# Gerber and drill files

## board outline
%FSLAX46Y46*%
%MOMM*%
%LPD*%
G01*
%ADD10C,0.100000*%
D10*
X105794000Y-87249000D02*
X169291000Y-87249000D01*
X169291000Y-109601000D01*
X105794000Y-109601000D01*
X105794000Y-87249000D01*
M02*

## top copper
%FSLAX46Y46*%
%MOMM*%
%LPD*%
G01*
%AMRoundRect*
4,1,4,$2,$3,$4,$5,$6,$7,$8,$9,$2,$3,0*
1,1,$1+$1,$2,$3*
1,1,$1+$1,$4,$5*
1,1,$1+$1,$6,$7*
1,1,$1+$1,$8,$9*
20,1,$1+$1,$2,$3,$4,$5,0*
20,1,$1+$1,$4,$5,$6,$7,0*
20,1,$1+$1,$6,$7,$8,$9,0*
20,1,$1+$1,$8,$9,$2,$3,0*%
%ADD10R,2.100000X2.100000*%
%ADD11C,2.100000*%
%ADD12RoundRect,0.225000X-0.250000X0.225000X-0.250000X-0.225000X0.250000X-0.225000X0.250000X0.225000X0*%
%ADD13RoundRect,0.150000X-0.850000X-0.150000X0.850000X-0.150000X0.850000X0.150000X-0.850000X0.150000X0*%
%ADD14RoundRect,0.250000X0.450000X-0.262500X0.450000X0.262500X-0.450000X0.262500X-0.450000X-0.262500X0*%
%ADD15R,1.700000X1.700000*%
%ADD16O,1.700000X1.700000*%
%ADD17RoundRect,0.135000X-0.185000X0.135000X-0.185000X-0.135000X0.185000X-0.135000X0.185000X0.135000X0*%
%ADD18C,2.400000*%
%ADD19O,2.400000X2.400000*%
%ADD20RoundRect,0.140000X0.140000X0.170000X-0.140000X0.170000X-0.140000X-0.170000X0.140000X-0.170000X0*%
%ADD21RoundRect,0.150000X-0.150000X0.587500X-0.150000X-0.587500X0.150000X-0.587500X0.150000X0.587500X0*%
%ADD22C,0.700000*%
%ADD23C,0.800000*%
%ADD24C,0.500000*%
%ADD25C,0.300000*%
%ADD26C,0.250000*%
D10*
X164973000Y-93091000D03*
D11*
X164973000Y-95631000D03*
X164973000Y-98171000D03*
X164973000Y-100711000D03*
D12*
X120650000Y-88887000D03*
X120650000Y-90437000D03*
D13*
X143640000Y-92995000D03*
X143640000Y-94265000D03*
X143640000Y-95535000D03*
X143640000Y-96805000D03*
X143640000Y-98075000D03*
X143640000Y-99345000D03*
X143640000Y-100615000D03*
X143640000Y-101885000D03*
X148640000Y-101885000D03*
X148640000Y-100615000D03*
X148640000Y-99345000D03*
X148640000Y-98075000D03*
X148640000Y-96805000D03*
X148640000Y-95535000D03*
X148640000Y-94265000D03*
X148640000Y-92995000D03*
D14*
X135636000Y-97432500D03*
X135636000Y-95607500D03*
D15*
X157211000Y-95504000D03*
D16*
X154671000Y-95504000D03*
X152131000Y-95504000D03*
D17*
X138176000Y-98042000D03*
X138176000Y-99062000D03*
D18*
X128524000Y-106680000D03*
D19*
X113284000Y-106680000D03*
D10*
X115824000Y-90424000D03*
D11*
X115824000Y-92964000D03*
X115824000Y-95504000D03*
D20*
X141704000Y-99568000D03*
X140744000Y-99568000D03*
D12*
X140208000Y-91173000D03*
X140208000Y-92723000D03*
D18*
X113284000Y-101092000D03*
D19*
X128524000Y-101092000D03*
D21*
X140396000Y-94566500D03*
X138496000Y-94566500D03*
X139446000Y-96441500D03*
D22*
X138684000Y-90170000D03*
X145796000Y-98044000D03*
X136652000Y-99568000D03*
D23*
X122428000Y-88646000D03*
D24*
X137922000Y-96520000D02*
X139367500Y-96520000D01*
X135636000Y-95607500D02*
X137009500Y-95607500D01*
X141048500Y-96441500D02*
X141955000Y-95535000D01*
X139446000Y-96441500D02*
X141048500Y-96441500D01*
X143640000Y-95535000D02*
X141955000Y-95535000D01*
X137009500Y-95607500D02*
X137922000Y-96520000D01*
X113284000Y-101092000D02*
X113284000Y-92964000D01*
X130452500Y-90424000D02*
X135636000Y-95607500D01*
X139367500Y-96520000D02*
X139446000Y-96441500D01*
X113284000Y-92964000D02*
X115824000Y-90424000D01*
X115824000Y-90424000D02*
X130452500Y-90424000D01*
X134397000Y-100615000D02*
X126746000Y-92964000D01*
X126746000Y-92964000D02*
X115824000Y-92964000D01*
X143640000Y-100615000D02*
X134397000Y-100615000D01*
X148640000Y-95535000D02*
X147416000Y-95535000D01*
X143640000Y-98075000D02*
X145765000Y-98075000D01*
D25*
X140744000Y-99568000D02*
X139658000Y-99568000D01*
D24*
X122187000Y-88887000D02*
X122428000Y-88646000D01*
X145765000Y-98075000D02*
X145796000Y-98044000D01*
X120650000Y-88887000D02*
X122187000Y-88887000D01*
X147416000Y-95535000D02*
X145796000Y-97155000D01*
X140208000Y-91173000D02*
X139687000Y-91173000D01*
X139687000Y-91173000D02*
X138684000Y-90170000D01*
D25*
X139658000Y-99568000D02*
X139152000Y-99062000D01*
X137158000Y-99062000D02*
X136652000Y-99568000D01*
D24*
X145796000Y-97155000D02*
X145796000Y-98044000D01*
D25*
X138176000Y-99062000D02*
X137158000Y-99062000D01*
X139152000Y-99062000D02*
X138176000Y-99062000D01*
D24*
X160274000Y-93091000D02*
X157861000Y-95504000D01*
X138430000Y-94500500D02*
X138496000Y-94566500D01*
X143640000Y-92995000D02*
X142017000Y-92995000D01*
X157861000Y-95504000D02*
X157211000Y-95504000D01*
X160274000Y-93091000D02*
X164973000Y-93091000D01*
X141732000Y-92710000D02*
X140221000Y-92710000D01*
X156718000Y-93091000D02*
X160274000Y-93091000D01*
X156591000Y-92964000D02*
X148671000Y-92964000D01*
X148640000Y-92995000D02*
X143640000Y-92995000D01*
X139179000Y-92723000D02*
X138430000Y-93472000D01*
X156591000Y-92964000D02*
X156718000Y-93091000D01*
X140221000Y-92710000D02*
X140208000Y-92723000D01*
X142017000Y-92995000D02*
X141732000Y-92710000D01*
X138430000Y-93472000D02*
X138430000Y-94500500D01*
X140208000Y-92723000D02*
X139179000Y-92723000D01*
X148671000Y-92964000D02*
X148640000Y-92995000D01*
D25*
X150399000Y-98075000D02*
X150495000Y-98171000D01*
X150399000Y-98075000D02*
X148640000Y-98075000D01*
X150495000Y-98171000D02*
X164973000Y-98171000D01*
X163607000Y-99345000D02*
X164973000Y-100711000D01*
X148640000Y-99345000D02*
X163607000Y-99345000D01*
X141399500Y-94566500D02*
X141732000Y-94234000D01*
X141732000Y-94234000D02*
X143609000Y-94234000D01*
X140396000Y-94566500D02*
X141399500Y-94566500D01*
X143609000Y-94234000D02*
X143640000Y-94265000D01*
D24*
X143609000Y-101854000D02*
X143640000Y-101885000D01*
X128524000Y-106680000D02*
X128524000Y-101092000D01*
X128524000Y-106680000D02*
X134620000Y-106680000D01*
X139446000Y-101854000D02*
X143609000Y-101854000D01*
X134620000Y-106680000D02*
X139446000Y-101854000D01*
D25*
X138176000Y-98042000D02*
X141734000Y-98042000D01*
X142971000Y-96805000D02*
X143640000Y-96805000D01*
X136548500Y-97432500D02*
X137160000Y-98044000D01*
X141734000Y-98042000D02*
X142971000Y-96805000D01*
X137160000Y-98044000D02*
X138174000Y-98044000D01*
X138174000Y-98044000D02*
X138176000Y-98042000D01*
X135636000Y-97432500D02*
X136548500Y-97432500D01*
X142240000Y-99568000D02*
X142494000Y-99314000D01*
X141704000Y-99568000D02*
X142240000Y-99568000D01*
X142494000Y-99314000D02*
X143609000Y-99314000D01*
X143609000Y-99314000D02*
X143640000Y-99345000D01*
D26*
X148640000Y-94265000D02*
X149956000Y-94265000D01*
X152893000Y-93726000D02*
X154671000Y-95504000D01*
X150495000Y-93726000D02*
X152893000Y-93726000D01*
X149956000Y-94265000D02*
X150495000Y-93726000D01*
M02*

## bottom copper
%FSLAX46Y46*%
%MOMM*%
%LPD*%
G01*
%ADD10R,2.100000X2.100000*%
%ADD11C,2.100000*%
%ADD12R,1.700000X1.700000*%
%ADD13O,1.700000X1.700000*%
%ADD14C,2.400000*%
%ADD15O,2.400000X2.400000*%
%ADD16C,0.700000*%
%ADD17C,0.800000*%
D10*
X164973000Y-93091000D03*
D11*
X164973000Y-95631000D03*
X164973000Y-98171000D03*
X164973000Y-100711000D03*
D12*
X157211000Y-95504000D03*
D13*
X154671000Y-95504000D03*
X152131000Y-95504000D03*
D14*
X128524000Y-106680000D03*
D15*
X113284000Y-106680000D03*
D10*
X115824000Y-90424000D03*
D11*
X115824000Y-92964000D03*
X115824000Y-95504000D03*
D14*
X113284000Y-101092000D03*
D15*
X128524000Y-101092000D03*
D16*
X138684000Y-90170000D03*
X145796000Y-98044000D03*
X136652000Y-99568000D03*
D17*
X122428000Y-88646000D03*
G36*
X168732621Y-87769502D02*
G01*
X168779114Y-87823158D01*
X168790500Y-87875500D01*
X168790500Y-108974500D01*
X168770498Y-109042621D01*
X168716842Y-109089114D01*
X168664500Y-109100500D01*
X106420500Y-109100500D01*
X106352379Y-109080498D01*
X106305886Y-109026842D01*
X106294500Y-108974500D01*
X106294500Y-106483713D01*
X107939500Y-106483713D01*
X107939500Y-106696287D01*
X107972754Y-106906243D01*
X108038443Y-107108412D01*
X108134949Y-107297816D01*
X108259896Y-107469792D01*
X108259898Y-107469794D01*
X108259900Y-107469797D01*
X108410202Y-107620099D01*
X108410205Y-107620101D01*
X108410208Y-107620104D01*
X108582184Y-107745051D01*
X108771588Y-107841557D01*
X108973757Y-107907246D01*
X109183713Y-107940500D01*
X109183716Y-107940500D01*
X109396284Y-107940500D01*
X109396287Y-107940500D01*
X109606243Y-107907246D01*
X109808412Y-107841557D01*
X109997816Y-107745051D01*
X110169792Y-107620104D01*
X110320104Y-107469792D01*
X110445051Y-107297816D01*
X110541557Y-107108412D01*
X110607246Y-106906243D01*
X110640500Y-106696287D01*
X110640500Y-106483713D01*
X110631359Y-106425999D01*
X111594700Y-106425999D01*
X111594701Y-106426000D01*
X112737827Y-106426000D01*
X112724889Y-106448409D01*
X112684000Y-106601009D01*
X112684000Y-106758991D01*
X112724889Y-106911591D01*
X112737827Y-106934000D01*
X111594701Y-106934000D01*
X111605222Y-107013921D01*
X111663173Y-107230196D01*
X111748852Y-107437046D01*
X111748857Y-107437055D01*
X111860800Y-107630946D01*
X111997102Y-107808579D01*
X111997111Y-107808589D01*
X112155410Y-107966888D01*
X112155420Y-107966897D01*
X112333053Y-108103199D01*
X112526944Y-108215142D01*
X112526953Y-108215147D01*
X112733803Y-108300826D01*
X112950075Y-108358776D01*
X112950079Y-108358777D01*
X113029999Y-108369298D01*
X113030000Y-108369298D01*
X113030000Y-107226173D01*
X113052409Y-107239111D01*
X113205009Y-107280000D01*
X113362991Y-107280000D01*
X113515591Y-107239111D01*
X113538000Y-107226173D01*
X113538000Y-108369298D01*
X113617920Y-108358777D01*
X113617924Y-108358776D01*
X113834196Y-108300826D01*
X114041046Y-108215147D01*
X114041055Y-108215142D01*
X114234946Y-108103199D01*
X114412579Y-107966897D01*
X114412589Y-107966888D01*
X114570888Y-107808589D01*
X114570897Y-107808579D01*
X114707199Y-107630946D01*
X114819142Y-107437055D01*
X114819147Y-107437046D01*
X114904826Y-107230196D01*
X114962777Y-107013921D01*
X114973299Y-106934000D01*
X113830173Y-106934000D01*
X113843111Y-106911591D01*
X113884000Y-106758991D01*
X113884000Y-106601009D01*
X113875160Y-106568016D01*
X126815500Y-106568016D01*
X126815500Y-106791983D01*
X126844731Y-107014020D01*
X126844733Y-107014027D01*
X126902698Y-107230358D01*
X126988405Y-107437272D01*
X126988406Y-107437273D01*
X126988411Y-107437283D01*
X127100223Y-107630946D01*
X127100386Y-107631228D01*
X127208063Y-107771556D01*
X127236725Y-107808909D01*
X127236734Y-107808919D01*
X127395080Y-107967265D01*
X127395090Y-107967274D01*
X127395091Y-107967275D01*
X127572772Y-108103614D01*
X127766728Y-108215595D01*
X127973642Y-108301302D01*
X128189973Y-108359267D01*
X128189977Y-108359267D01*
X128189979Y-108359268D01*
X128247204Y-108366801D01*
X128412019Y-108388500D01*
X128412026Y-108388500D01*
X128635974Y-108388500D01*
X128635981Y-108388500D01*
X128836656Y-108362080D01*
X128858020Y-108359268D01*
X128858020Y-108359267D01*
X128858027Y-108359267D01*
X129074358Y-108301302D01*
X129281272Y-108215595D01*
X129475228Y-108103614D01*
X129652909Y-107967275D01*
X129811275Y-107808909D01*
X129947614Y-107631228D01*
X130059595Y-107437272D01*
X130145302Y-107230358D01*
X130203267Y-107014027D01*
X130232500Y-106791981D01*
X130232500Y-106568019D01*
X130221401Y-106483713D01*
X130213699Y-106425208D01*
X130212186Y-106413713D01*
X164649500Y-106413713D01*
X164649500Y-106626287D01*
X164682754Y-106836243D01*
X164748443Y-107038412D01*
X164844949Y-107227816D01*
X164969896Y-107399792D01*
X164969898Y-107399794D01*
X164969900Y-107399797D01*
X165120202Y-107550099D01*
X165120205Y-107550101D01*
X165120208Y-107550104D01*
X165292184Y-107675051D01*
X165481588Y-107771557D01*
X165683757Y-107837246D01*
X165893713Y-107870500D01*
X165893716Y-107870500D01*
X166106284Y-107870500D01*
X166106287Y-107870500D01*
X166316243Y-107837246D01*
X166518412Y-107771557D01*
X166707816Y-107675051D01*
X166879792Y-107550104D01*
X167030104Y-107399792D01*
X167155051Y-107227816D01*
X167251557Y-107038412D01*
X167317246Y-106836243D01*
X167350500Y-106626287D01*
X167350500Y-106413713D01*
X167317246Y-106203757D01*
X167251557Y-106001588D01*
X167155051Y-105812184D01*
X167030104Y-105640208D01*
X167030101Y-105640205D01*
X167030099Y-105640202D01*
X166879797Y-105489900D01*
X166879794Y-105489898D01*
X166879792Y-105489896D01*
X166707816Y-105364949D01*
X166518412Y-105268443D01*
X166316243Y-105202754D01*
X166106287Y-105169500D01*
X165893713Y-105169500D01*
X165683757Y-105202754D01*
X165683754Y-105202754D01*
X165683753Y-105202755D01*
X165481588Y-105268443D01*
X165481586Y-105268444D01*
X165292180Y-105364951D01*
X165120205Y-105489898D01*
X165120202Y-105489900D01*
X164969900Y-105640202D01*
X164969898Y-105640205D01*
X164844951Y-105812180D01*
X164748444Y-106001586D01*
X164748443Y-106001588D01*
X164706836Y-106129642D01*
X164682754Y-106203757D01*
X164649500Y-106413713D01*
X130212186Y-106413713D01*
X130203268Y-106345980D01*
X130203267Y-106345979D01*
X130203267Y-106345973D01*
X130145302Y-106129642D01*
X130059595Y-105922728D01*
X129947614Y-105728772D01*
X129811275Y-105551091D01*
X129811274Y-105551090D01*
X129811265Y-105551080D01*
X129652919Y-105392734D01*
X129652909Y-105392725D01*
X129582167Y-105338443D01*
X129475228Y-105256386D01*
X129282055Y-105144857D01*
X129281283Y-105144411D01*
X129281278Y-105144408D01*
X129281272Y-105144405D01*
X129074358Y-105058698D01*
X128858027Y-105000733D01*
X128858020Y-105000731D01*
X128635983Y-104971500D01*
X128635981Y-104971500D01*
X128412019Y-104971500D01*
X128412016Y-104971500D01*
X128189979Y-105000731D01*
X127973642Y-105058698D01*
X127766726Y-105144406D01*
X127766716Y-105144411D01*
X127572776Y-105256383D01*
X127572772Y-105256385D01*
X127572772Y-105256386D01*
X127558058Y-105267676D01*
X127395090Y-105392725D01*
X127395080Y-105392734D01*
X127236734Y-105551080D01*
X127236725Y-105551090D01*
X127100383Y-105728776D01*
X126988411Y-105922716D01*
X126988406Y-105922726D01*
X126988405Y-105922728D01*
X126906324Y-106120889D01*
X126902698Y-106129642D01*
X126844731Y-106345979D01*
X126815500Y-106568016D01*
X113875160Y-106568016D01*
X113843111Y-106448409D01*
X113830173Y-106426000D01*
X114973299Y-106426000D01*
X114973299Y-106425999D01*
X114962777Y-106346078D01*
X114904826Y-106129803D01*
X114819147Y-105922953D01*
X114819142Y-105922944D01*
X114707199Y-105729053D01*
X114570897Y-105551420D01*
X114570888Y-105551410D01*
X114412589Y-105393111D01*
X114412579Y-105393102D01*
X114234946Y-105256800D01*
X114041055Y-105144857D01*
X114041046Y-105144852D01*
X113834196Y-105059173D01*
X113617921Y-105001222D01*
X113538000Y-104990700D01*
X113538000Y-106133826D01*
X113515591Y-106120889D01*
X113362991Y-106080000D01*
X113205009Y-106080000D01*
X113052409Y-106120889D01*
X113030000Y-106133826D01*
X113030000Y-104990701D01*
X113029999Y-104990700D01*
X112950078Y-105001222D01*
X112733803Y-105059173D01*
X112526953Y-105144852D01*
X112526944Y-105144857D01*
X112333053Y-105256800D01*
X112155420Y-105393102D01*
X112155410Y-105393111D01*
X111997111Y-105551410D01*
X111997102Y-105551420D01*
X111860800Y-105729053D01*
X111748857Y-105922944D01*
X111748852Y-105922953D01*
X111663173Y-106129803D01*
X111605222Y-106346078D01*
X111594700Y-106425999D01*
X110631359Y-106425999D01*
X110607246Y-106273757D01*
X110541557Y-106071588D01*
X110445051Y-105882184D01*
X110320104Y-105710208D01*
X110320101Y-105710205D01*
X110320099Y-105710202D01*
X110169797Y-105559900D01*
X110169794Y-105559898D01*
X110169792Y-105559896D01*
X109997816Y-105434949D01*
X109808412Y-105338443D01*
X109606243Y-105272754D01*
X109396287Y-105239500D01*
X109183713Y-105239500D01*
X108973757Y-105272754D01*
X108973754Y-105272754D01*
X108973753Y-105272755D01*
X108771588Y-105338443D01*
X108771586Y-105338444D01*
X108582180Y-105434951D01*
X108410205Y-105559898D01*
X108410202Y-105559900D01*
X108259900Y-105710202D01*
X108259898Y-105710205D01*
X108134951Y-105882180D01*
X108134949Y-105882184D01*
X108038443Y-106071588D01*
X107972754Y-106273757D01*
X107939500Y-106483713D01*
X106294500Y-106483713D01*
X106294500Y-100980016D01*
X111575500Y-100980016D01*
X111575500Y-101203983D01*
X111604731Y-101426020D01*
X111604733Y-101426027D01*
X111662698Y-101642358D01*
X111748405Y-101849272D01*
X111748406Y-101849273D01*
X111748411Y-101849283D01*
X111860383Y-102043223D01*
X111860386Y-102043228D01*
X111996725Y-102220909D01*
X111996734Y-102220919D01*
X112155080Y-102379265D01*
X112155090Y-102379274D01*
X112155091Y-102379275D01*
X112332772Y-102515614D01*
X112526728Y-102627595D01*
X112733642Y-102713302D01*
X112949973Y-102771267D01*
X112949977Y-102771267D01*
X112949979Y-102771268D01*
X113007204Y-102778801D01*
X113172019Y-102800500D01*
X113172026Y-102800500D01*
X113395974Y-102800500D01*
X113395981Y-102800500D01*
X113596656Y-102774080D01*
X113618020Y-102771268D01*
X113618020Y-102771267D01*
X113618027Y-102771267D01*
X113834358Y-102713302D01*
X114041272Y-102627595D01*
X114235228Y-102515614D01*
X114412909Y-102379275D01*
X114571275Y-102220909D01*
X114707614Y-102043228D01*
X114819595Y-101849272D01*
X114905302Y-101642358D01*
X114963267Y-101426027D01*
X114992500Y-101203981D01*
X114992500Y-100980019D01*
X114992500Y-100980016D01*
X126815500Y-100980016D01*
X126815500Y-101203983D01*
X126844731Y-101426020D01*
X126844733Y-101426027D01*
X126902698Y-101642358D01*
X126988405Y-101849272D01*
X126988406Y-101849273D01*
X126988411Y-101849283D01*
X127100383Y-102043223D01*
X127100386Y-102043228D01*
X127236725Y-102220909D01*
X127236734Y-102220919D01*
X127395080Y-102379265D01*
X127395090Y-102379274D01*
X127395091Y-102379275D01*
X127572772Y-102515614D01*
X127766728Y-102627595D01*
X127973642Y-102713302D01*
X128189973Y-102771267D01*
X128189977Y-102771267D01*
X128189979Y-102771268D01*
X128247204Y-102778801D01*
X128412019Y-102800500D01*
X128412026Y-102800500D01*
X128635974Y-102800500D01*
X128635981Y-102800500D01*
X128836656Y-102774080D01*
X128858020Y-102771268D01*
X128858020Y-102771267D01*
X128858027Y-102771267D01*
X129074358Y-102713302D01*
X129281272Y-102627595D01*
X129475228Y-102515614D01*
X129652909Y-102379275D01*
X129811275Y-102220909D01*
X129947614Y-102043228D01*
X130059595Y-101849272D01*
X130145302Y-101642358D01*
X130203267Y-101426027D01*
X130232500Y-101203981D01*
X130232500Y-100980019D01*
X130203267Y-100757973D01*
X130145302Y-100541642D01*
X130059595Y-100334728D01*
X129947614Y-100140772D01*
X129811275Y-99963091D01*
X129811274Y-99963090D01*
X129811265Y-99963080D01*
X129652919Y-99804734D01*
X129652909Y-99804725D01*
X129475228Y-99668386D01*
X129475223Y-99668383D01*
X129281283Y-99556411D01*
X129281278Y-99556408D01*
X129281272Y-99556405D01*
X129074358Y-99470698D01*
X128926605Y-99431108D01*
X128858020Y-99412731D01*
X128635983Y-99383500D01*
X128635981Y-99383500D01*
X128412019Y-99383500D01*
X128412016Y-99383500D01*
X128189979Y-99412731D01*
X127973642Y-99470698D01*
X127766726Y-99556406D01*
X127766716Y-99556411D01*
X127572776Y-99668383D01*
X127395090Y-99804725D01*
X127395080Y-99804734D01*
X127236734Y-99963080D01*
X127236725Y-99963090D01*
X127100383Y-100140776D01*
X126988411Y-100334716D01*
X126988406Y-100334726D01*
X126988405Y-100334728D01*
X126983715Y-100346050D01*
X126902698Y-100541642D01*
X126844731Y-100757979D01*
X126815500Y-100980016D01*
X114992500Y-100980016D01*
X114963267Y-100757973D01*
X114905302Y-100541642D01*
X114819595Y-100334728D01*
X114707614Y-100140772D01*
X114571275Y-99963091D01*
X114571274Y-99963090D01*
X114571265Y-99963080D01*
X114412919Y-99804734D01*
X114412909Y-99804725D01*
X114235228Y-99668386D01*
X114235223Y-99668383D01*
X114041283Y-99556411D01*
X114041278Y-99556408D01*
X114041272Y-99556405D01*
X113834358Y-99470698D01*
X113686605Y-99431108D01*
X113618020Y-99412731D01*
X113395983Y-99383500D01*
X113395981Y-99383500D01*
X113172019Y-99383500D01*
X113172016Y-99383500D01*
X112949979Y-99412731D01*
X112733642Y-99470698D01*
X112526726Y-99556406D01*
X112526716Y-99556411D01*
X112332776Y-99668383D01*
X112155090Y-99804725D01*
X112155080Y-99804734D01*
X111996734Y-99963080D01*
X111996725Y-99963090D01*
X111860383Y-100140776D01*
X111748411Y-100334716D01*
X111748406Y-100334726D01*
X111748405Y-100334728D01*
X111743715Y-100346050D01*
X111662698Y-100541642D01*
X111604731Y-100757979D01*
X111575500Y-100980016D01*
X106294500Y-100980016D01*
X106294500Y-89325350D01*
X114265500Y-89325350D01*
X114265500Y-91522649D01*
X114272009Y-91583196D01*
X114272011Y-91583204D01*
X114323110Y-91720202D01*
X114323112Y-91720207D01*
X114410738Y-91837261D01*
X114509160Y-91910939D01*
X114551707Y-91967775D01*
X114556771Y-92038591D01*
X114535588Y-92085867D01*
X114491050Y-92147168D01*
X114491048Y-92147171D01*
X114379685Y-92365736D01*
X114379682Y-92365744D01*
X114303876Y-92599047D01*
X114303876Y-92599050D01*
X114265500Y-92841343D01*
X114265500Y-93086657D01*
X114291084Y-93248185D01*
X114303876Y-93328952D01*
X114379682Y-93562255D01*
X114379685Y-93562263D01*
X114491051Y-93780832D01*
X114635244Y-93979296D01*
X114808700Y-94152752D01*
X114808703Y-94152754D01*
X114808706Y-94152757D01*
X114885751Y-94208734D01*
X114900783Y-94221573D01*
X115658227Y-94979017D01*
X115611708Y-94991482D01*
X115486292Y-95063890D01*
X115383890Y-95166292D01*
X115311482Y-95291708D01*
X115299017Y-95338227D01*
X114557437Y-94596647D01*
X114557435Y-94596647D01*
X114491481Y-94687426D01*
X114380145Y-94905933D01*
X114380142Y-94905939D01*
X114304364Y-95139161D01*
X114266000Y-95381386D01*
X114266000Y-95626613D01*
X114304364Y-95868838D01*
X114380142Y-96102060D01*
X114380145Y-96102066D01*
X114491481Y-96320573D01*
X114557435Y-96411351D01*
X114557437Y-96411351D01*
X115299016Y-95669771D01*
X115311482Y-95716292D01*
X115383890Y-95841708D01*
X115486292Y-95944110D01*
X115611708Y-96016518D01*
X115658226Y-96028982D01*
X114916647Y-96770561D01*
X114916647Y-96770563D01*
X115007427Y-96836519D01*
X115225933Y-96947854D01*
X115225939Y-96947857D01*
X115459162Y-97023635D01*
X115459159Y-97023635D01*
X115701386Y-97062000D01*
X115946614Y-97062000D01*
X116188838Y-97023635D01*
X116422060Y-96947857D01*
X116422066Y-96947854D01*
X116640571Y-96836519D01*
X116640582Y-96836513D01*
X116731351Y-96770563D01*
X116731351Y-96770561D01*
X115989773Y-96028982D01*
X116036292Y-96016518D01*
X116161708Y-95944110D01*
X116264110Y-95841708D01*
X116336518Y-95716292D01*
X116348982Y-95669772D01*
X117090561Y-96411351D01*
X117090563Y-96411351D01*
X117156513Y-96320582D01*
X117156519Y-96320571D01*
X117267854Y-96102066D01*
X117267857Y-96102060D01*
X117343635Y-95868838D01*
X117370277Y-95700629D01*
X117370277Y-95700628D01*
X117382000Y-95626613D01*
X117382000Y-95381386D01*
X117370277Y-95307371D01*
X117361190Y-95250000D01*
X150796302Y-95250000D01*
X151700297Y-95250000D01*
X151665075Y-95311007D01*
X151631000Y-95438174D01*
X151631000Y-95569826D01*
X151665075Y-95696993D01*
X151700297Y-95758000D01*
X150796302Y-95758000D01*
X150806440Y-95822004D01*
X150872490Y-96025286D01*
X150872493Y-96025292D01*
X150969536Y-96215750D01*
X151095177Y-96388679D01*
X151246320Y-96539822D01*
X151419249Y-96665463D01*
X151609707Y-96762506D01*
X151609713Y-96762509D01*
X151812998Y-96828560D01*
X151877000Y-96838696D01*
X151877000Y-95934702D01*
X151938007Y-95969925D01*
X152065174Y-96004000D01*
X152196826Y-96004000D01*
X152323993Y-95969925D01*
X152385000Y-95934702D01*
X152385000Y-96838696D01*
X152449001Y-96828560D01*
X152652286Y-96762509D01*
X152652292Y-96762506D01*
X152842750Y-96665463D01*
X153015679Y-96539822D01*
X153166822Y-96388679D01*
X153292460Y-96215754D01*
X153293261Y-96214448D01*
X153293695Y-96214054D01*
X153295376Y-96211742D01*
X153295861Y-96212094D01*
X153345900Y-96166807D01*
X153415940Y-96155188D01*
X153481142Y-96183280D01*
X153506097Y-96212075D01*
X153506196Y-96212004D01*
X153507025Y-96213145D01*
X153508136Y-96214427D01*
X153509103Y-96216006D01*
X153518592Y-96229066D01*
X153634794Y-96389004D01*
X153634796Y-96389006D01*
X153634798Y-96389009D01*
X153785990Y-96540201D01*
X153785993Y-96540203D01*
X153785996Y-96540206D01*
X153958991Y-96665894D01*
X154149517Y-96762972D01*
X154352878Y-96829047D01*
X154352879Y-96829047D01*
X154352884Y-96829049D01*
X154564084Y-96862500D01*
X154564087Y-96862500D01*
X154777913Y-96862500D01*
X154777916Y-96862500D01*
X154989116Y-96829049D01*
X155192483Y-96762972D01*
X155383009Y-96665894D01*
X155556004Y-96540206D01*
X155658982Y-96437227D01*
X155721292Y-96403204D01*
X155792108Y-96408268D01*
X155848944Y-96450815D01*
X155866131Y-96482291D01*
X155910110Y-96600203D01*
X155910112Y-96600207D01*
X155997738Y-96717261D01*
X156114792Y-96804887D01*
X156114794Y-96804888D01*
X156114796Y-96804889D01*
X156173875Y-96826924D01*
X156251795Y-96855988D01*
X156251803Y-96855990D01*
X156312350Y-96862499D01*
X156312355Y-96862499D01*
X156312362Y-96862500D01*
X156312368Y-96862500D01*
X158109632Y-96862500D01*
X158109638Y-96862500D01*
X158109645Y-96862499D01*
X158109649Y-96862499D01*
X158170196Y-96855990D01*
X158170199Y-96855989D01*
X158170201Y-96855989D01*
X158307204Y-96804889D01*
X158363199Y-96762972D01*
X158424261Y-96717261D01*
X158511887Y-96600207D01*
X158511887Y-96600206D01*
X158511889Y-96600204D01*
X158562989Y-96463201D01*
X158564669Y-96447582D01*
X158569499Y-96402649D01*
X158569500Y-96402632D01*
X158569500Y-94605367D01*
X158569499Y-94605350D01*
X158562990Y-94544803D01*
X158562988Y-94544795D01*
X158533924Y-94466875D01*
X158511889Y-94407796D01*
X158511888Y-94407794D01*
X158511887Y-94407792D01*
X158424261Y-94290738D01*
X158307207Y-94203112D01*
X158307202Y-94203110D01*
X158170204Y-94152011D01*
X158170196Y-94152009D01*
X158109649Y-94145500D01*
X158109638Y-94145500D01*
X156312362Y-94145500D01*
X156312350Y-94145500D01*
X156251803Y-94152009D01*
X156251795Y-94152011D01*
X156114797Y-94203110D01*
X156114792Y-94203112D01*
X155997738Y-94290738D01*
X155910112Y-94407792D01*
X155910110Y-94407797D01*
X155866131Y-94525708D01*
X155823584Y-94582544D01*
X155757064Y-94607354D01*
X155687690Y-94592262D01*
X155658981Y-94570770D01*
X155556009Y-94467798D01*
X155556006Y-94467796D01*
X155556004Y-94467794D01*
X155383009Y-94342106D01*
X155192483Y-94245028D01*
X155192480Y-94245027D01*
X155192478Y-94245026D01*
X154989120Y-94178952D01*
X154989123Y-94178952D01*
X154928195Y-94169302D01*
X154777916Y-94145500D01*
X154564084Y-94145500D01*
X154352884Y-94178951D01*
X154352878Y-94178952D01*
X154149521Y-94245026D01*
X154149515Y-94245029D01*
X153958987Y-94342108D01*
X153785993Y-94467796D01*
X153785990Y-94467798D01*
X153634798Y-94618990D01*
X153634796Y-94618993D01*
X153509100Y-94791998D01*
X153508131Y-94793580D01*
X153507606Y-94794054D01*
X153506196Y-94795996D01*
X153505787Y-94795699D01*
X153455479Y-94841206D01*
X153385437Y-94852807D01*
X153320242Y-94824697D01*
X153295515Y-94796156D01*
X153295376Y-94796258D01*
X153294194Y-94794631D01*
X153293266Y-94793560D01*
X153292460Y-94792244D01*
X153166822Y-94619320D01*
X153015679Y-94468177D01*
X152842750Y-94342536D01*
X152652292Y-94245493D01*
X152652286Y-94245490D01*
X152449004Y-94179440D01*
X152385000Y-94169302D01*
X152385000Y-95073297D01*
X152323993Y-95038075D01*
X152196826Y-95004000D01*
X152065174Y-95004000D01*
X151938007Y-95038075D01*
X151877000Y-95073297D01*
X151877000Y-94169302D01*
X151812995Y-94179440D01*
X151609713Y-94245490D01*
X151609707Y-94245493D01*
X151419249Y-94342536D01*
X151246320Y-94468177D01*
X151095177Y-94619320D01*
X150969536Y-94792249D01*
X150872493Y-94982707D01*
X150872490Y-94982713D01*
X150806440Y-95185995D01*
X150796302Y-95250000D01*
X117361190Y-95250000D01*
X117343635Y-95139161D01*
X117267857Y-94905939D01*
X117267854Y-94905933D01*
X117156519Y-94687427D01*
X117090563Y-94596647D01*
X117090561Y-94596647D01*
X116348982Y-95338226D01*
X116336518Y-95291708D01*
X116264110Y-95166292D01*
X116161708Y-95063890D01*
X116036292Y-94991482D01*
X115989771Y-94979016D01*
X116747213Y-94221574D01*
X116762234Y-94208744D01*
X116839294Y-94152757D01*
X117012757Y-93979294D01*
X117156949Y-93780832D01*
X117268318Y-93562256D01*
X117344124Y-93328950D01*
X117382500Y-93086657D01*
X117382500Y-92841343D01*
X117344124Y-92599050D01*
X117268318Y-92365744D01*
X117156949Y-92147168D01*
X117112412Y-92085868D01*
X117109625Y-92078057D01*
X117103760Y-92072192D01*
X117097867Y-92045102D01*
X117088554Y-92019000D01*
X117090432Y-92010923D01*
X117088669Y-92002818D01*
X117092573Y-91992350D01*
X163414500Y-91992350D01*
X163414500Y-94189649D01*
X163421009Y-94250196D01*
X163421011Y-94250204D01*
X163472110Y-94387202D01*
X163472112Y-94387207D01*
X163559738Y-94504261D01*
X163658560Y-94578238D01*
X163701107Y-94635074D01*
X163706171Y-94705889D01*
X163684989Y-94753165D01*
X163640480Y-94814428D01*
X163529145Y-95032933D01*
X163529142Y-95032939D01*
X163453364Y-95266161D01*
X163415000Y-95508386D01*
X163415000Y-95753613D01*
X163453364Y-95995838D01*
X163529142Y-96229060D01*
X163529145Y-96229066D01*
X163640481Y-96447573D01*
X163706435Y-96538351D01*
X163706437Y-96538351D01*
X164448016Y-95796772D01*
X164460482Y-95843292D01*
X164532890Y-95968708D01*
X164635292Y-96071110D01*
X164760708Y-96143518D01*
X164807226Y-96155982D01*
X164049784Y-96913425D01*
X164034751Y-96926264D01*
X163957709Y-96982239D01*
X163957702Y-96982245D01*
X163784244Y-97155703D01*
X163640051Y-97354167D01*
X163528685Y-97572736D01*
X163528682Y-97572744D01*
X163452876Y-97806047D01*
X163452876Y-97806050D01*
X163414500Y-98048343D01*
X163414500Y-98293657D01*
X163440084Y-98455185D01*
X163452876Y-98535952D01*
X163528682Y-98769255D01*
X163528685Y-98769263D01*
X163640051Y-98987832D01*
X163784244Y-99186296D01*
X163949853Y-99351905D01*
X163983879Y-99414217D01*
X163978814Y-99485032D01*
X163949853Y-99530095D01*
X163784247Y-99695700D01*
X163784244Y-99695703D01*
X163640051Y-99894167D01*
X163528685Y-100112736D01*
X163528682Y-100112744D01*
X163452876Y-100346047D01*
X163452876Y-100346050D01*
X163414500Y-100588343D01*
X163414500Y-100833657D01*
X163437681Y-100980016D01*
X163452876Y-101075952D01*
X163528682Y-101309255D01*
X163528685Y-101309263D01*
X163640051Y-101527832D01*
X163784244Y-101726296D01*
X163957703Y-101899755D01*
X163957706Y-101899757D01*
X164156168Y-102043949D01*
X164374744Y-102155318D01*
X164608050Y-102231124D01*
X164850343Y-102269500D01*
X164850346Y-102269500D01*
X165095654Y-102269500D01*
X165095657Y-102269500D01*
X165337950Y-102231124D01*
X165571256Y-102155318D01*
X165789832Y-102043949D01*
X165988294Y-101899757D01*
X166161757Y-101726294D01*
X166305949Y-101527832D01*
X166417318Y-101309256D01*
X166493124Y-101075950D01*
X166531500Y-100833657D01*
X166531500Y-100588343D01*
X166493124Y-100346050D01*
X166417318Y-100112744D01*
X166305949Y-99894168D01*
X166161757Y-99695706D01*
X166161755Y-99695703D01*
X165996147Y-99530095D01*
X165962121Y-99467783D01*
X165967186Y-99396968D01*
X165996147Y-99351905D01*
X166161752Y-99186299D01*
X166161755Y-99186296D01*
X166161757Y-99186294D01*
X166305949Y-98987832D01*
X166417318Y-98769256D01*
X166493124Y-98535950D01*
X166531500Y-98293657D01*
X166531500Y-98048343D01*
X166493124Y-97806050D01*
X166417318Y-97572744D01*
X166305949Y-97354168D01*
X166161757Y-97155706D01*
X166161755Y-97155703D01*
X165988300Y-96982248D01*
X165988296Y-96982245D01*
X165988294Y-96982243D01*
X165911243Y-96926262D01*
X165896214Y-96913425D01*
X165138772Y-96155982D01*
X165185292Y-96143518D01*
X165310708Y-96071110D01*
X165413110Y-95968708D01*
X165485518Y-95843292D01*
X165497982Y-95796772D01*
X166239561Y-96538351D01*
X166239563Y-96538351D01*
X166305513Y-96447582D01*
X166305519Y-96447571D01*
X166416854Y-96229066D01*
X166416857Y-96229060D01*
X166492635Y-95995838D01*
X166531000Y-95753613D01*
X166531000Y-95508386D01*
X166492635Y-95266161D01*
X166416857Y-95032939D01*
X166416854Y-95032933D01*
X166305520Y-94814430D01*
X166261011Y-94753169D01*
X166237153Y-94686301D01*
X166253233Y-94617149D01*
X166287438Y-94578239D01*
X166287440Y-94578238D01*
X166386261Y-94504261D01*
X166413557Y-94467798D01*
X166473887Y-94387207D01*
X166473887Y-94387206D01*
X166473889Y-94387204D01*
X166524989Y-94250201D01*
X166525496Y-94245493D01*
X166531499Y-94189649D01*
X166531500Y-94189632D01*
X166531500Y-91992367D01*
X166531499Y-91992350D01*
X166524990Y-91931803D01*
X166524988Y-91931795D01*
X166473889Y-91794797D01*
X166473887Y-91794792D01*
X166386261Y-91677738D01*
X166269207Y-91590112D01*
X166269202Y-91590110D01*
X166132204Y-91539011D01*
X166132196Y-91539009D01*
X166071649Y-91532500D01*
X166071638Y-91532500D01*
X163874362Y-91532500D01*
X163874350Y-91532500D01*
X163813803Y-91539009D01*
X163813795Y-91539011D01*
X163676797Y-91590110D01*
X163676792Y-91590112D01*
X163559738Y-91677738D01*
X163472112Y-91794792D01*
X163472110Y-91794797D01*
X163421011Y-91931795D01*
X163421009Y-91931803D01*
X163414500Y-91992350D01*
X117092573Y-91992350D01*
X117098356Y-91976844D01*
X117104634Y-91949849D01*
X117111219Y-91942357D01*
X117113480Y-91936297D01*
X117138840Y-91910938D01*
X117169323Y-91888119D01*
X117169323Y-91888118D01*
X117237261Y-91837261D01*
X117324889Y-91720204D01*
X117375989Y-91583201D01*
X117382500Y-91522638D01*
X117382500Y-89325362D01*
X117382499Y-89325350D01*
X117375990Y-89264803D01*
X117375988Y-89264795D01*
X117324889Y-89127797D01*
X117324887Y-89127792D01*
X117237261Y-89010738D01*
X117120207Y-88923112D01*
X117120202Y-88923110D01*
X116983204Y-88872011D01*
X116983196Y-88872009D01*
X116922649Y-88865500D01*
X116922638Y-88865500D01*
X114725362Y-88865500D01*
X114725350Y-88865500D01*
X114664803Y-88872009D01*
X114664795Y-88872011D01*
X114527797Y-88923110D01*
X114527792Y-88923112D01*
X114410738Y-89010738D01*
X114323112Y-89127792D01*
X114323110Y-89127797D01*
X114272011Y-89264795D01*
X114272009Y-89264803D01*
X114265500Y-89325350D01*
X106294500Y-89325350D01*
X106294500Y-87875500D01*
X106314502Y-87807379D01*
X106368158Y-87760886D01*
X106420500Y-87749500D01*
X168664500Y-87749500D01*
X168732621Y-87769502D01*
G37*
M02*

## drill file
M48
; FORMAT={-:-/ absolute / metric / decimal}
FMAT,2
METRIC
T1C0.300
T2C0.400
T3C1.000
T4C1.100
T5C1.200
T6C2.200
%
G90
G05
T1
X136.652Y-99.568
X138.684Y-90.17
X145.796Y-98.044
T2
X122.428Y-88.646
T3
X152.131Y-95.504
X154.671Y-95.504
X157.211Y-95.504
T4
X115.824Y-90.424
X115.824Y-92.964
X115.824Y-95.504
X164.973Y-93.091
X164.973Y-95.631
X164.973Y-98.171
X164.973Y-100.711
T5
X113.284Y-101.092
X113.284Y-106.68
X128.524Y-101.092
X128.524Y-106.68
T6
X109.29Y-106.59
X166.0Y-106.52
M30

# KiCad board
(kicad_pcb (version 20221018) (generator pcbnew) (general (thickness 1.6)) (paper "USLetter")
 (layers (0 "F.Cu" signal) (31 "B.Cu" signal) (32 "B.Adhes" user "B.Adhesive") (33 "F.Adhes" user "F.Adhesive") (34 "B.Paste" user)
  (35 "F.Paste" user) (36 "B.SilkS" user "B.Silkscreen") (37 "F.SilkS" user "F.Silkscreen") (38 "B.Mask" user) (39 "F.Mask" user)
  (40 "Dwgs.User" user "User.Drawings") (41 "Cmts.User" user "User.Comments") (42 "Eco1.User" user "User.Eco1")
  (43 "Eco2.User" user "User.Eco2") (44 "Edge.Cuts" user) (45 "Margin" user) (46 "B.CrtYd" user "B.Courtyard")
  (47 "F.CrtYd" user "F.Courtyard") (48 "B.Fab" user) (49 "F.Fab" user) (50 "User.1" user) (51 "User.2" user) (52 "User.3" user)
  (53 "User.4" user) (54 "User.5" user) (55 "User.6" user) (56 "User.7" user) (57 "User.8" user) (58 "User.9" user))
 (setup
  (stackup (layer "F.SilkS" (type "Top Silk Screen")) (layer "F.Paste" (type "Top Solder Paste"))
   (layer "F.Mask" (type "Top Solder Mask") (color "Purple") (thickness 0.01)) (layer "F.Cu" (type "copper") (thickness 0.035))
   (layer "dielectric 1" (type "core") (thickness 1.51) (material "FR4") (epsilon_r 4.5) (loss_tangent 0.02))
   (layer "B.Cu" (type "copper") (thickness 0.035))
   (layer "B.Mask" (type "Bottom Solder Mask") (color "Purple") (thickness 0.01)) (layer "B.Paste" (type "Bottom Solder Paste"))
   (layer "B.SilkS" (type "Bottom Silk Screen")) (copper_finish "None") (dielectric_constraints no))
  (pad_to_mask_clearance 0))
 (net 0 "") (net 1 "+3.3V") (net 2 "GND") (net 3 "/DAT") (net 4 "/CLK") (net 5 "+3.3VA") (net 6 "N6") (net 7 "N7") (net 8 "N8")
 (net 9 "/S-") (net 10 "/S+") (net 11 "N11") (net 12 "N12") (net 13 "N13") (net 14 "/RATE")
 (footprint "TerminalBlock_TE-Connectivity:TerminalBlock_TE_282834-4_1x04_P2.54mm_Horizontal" (layer "F.Cu") (at 164.973 93.091 -90)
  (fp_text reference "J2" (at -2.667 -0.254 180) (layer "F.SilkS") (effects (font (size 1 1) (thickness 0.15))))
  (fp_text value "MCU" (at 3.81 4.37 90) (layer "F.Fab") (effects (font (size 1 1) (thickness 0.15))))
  (pad "1" thru_hole rect (at 0 0 270) (size 2.1 2.1) (drill 1.1) (layers "*.Cu" "*.Mask") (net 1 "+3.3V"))
  (pad "2" thru_hole circle (at 2.54 0 270) (size 2.1 2.1) (drill 1.1) (layers "*.Cu" "*.Mask") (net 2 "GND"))
  (pad "3" thru_hole circle (at 5.08 0 270) (size 2.1 2.1) (drill 1.1) (layers "*.Cu" "*.Mask") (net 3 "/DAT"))
  (pad "4" thru_hole circle (at 7.62 0 270) (size 2.1 2.1) (drill 1.1) (layers "*.Cu" "*.Mask") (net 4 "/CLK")))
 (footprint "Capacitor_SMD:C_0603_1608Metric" (layer "F.Cu") (at 120.65 89.662 -90)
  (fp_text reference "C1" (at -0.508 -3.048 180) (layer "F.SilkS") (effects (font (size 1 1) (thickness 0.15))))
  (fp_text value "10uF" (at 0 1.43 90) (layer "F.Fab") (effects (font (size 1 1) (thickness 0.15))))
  (pad "1" smd roundrect (at -0.775 0 270) (size 0.9 0.95) (layers "F.Cu" "F.Paste" "F.Mask") (roundrect_rratio 0.25) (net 2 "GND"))
  (pad "2" smd roundrect (at 0.775 0 270) (size 0.9 0.95) (layers "F.Cu" "F.Paste" "F.Mask") (roundrect_rratio 0.25) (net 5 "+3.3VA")))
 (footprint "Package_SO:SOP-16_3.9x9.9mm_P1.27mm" (layer "F.Cu") (at 146.14 97.44)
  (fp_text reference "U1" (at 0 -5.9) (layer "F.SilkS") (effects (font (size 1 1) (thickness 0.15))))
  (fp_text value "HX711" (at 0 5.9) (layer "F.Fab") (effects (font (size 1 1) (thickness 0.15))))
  (pad "1" smd roundrect (at -2.5 -4.445) (size 2 0.6) (layers "F.Cu" "F.Paste" "F.Mask") (roundrect_rratio 0.25) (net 1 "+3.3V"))
  (pad "2" smd roundrect (at -2.5 -3.175) (size 2 0.6) (layers "F.Cu" "F.Paste" "F.Mask") (roundrect_rratio 0.25) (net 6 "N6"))
  (pad "3" smd roundrect (at -2.5 -1.905) (size 2 0.6) (layers "F.Cu" "F.Paste" "F.Mask") (roundrect_rratio 0.25) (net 5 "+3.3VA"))
  (pad "4" smd roundrect (at -2.5 -0.635) (size 2 0.6) (layers "F.Cu" "F.Paste" "F.Mask") (roundrect_rratio 0.25) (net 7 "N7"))
  (pad "5" smd roundrect (at -2.5 0.635) (size 2 0.6) (layers "F.Cu" "F.Paste" "F.Mask") (roundrect_rratio 0.25) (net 2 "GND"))
  (pad "6" smd roundrect (at -2.5 1.905) (size 2 0.6) (layers "F.Cu" "F.Paste" "F.Mask") (roundrect_rratio 0.25) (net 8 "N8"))
  (pad "7" smd roundrect (at -2.5 3.175) (size 2 0.6) (layers "F.Cu" "F.Paste" "F.Mask") (roundrect_rratio 0.25) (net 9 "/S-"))
  (pad "8" smd roundrect (at -2.5 4.445) (size 2 0.6) (layers "F.Cu" "F.Paste" "F.Mask") (roundrect_rratio 0.25) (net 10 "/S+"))
  (pad "9" smd roundrect (at 2.5 4.445) (size 2 0.6) (layers "F.Cu" "F.Paste" "F.Mask") (roundrect_rratio 0.25) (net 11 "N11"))
  (pad "10" smd roundrect (at 2.5 3.175) (size 2 0.6) (layers "F.Cu" "F.Paste" "F.Mask") (roundrect_rratio 0.25) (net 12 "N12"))
  (pad "11" smd roundrect (at 2.5 1.905) (size 2 0.6) (layers "F.Cu" "F.Paste" "F.Mask") (roundrect_rratio 0.25) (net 4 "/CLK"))
  (pad "12" smd roundrect (at 2.5 0.635) (size 2 0.6) (layers "F.Cu" "F.Paste" "F.Mask") (roundrect_rratio 0.25) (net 3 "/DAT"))
  (pad "13" smd roundrect (at 2.5 -0.635) (size 2 0.6) (layers "F.Cu" "F.Paste" "F.Mask") (roundrect_rratio 0.25) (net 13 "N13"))
  (pad "14" smd roundrect (at 2.5 -1.905) (size 2 0.6) (layers "F.Cu" "F.Paste" "F.Mask") (roundrect_rratio 0.25) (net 2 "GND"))
  (pad "15" smd roundrect (at 2.5 -3.175) (size 2 0.6) (layers "F.Cu" "F.Paste" "F.Mask") (roundrect_rratio 0.25) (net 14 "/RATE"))
  (pad "16" smd roundrect (at 2.5 -4.445) (size 2 0.6) (layers "F.Cu" "F.Paste" "F.Mask") (roundrect_rratio 0.25) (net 1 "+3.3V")))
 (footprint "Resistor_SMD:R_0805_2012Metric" (layer "F.Cu") (at 135.636 96.52 90)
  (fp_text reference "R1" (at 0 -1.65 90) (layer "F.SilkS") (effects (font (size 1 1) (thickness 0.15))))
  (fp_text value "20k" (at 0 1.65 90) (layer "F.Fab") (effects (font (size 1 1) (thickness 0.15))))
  (pad "1" smd roundrect (at -0.9125 0 90) (size 1.025 1.4) (layers "F.Cu" "F.Paste" "F.Mask") (roundrect_rratio 0.243902439) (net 7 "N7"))
  (pad "2" smd roundrect (at 0.9125 0 90) (size 1.025 1.4) (layers "F.Cu" "F.Paste" "F.Mask") (roundrect_rratio 0.243902439)
   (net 5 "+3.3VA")))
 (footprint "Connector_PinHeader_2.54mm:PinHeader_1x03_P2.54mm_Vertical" (layer "F.Cu") (at 157.211 95.504 -90)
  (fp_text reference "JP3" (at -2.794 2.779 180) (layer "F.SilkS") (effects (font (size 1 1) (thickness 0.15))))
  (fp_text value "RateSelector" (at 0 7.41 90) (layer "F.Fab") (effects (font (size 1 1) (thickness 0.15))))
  (pad "1" thru_hole rect (at 0 0 270) (size 1.7 1.7) (drill 1) (layers "*.Cu" "*.Mask") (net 1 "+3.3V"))
  (pad "2" thru_hole oval (at 0 2.54 270) (size 1.7 1.7) (drill 1) (layers "*.Cu" "*.Mask") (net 14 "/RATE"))
  (pad "3" thru_hole oval (at 0 5.08 270) (size 1.7 1.7) (drill 1) (layers "*.Cu" "*.Mask") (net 2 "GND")))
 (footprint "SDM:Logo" (layer "F.Cu") (at 135.255 105.029)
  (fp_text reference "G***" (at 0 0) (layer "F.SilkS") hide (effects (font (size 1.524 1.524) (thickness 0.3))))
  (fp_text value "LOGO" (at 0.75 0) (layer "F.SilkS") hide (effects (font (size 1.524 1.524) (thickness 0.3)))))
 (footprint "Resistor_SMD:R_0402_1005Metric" (layer "F.Cu") (at 138.176 98.552 -90)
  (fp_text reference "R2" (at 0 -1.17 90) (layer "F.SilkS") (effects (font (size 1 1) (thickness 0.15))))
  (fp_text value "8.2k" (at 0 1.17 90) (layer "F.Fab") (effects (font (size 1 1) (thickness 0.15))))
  (pad "1" smd roundrect (at -0.51 0 270) (size 0.54 0.64) (layers "F.Cu" "F.Paste" "F.Mask") (roundrect_rratio 0.25) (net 7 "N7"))
  (pad "2" smd roundrect (at 0.51 0 270) (size 0.54 0.64) (layers "F.Cu" "F.Paste" "F.Mask") (roundrect_rratio 0.25) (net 2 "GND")))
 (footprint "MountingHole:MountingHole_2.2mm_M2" (layer "F.Cu") (at 109.29 106.59)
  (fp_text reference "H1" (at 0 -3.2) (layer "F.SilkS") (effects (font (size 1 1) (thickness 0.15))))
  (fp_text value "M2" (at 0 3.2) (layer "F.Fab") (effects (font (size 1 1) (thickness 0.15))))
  (pad "" np_thru_hole circle (at 0 0) (size 2.2 2.2) (drill 2.2) (layers "*.Cu" "*.Mask")))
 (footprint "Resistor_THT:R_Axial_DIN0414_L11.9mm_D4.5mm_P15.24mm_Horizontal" (layer "F.Cu") (at 128.524 106.68 180)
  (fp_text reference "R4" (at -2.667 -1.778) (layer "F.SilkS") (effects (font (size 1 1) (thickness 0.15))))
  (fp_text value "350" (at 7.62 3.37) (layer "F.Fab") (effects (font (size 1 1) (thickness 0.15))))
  (pad "1" thru_hole circle (at 0 0 180) (size 2.4 2.4) (drill 1.2) (layers "*.Cu" "*.Mask") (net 10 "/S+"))
  (pad "2" thru_hole oval (at 15.24 0 180) (size 2.4 2.4) (drill 1.2) (layers "*.Cu" "*.Mask") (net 2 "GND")))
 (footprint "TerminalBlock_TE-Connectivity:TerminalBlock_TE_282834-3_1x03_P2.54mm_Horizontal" (layer "F.Cu") (at 115.824 90.424 -90)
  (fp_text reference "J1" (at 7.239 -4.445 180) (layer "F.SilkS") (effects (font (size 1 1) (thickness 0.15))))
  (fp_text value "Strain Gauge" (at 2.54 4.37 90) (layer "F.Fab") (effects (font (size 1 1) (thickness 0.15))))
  (pad "1" thru_hole rect (at 0 0 270) (size 2.1 2.1) (drill 1.1) (layers "*.Cu" "*.Mask") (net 5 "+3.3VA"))
  (pad "2" thru_hole circle (at 2.54 0 270) (size 2.1 2.1) (drill 1.1) (layers "*.Cu" "*.Mask") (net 9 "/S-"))
  (pad "3" thru_hole circle (at 5.08 0 270) (size 2.1 2.1) (drill 1.1) (layers "*.Cu" "*.Mask") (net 2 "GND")))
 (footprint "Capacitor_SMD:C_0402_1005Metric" (layer "F.Cu") (at 141.224 99.568 180)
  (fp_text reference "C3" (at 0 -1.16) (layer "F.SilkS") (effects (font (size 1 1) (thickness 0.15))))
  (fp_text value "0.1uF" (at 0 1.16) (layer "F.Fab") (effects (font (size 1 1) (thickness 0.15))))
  (pad "1" smd roundrect (at -0.48 0 180) (size 0.56 0.62) (layers "F.Cu" "F.Paste" "F.Mask") (roundrect_rratio 0.25) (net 8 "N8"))
  (pad "2" smd roundrect (at 0.48 0 180) (size 0.56 0.62) (layers "F.Cu" "F.Paste" "F.Mask") (roundrect_rratio 0.25) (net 2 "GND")))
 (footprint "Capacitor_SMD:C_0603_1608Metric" (layer "F.Cu") (at 140.208 91.948 -90)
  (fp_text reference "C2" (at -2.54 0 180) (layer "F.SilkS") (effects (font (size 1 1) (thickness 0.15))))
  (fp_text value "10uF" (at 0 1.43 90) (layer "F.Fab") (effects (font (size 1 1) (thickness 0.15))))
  (pad "1" smd roundrect (at -0.775 0 270) (size 0.9 0.95) (layers "F.Cu" "F.Paste" "F.Mask") (roundrect_rratio 0.25) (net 2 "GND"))
  (pad "2" smd roundrect (at 0.775 0 270) (size 0.9 0.95) (layers "F.Cu" "F.Paste" "F.Mask") (roundrect_rratio 0.25) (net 1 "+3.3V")))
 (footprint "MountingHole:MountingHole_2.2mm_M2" (layer "F.Cu") (at 166 106.52)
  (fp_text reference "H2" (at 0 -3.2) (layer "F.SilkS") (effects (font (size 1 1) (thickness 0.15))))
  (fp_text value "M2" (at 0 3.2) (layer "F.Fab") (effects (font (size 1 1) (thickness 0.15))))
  (pad "" np_thru_hole circle (at 0 0) (size 2.2 2.2) (drill 2.2) (layers "*.Cu" "*.Mask")))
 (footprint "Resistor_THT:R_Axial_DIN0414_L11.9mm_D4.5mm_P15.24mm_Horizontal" (layer "F.Cu") (at 113.284 101.092)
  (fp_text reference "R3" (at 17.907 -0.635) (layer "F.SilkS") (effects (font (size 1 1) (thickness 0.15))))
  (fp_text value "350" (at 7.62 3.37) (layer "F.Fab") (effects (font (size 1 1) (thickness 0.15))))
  (pad "1" thru_hole circle (at 0 0) (size 2.4 2.4) (drill 1.2) (layers "*.Cu" "*.Mask") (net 5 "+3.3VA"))
  (pad "2" thru_hole oval (at 15.24 0) (size 2.4 2.4) (drill 1.2) (layers "*.Cu" "*.Mask") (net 10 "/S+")))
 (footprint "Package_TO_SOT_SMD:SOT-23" (layer "F.Cu") (at 139.446 95.504 -90)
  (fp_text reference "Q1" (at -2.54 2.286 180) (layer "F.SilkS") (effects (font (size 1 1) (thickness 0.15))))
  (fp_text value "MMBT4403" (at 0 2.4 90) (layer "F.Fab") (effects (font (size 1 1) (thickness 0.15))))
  (pad "1" smd roundrect (at -0.9375 -0.95 270) (size 1.475 0.6) (layers "F.Cu" "F.Paste" "F.Mask") (roundrect_rratio 0.25) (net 6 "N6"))
  (pad "2" smd roundrect (at -0.9375 0.95 270) (size 1.475 0.6) (layers "F.Cu" "F.Paste" "F.Mask") (roundrect_rratio 0.25) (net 1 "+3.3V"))
  (pad "3" smd roundrect (at 0.9375 0 270) (size 1.475 0.6) (layers "F.Cu" "F.Paste" "F.Mask") (roundrect_rratio 0.25) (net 5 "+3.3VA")))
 (gr_rect (start 105.794 87.249) (end 169.291 109.601) (stroke (width 0.1) (type solid)) (fill none) (layer "Edge.Cuts"))
 (segment (start 137.922 96.52) (end 139.3675 96.52) (width 0.5) (layer "F.Cu") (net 5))
 (segment (start 135.636 95.6075) (end 137.0095 95.6075) (width 0.5) (layer "F.Cu") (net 5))
 (segment (start 141.0485 96.4415) (end 141.955 95.535) (width 0.5) (layer "F.Cu") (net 5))
 (segment (start 139.446 96.4415) (end 141.0485 96.4415) (width 0.5) (layer "F.Cu") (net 5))
 (segment (start 143.64 95.535) (end 141.955 95.535) (width 0.5) (layer "F.Cu") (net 5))
 (segment (start 137.0095 95.6075) (end 137.922 96.52) (width 0.5) (layer "F.Cu") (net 5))
 (segment (start 113.284 101.092) (end 113.284 92.964) (width 0.5) (layer "F.Cu") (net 5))
 (segment (start 130.4525 90.424) (end 135.636 95.6075) (width 0.5) (layer "F.Cu") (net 5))
 (segment (start 139.3675 96.52) (end 139.446 96.4415) (width 0.5) (layer "F.Cu") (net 5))
 (segment (start 113.284 92.964) (end 115.824 90.424) (width 0.5) (layer "F.Cu") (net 5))
 (segment (start 115.824 90.424) (end 130.4525 90.424) (width 0.5) (layer "F.Cu") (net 5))
 (segment (start 134.397 100.615) (end 126.746 92.964) (width 0.5) (layer "F.Cu") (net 9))
 (segment (start 126.746 92.964) (end 115.824 92.964) (width 0.5) (layer "F.Cu") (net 9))
 (segment (start 143.64 100.615) (end 134.397 100.615) (width 0.5) (layer "F.Cu") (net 9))
 (segment (start 148.64 95.535) (end 147.416 95.535) (width 0.5) (layer "F.Cu") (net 2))
 (segment (start 143.64 98.075) (end 145.765 98.075) (width 0.5) (layer "F.Cu") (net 2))
 (segment (start 140.744 99.568) (end 139.658 99.568) (width 0.3) (layer "F.Cu") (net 2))
 (segment (start 122.187 88.887) (end 122.428 88.646) (width 0.5) (layer "F.Cu") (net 2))
 (segment (start 145.765 98.075) (end 145.796 98.044) (width 0.5) (layer "F.Cu") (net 2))
 (segment (start 120.65 88.887) (end 122.187 88.887) (width 0.5) (layer "F.Cu") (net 2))
 (segment (start 147.416 95.535) (end 145.796 97.155) (width 0.5) (layer "F.Cu") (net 2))
 (segment (start 140.208 91.173) (end 139.687 91.173) (width 0.5) (layer "F.Cu") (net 2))
 (segment (start 139.687 91.173) (end 138.684 90.17) (width 0.5) (layer "F.Cu") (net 2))
 (segment (start 139.658 99.568) (end 139.152 99.062) (width 0.3) (layer "F.Cu") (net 2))
 (segment (start 137.158 99.062) (end 136.652 99.568) (width 0.3) (layer "F.Cu") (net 2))
 (segment (start 145.796 97.155) (end 145.796 98.044) (width 0.5) (layer "F.Cu") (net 2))
 (segment (start 138.176 99.062) (end 137.158 99.062) (width 0.3) (layer "F.Cu") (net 2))
 (segment (start 139.152 99.062) (end 138.176 99.062) (width 0.3) (layer "F.Cu") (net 2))
 (via (at 138.684 90.17) (size 0.7) (drill 0.3) (layers "F.Cu" "B.Cu") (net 2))
 (via (at 145.796 98.044) (size 0.7) (drill 0.3) (layers "F.Cu" "B.Cu") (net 2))
 (via (at 136.652 99.568) (size 0.7) (drill 0.3) (layers "F.Cu" "B.Cu") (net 2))
 (via (at 122.428 88.646) (size 0.8) (drill 0.4) (layers "F.Cu" "B.Cu") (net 2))
 (segment (start 160.274 93.091) (end 157.861 95.504) (width 0.5) (layer "F.Cu") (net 1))
 (segment (start 138.43 94.5005) (end 138.496 94.5665) (width 0.5) (layer "F.Cu") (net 1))
 (segment (start 143.64 92.995) (end 142.017 92.995) (width 0.5) (layer "F.Cu") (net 1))
 (segment (start 157.861 95.504) (end 157.211 95.504) (width 0.5) (layer "F.Cu") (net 1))
 (segment (start 160.274 93.091) (end 164.973 93.091) (width 0.5) (layer "F.Cu") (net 1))
 (segment (start 141.732 92.71) (end 140.221 92.71) (width 0.5) (layer "F.Cu") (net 1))
 (segment (start 156.718 93.091) (end 160.274 93.091) (width 0.5) (layer "F.Cu") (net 1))
 (segment (start 156.591 92.964) (end 148.671 92.964) (width 0.5) (layer "F.Cu") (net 1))
 (segment (start 148.64 92.995) (end 143.64 92.995) (width 0.5) (layer "F.Cu") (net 1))
 (segment (start 139.179 92.723) (end 138.43 93.472) (width 0.5) (layer "F.Cu") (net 1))
 (segment (start 156.591 92.964) (end 156.718 93.091) (width 0.5) (layer "F.Cu") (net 1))
 (segment (start 140.221 92.71) (end 140.208 92.723) (width 0.5) (layer "F.Cu") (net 1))
 (segment (start 142.017 92.995) (end 141.732 92.71) (width 0.5) (layer "F.Cu") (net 1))
 (segment (start 138.43 93.472) (end 138.43 94.5005) (width 0.5) (layer "F.Cu") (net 1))
 (segment (start 140.208 92.723) (end 139.179 92.723) (width 0.5) (layer "F.Cu") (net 1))
 (segment (start 148.671 92.964) (end 148.64 92.995) (width 0.5) (layer "F.Cu") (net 1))
 (segment (start 150.399 98.075) (end 150.495 98.171) (width 0.3) (layer "F.Cu") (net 3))
 (segment (start 150.399 98.075) (end 148.64 98.075) (width 0.3) (layer "F.Cu") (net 3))
 (segment (start 150.495 98.171) (end 164.973 98.171) (width 0.3) (layer "F.Cu") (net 3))
 (segment (start 163.607 99.345) (end 164.973 100.711) (width 0.3) (layer "F.Cu") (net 4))
 (segment (start 148.64 99.345) (end 163.607 99.345) (width 0.3) (layer "F.Cu") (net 4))
 (segment (start 141.3995 94.5665) (end 141.732 94.234) (width 0.3) (layer "F.Cu") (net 6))
 (segment (start 141.732 94.234) (end 143.609 94.234) (width 0.3) (layer "F.Cu") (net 6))
 (segment (start 140.396 94.5665) (end 141.3995 94.5665) (width 0.3) (layer "F.Cu") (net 6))
 (segment (start 143.609 94.234) (end 143.64 94.265) (width 0.3) (layer "F.Cu") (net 6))
 (segment (start 143.609 101.854) (end 143.64 101.885) (width 0.5) (layer "F.Cu") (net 10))
 (segment (start 128.524 106.68) (end 128.524 101.092) (width 0.5) (layer "F.Cu") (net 10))
 (segment (start 128.524 106.68) (end 134.62 106.68) (width 0.5) (layer "F.Cu") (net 10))
 (segment (start 139.446 101.854) (end 143.609 101.854) (width 0.5) (layer "F.Cu") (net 10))
 (segment (start 134.62 106.68) (end 139.446 101.854) (width 0.5) (layer "F.Cu") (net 10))
 (segment (start 138.176 98.042) (end 141.734 98.042) (width 0.3) (layer "F.Cu") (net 7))
 (segment (start 142.971 96.805) (end 143.64 96.805) (width 0.3) (layer "F.Cu") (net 7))
 (segment (start 136.5485 97.4325) (end 137.16 98.044) (width 0.3) (layer "F.Cu") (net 7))
 (segment (start 141.734 98.042) (end 142.971 96.805) (width 0.3) (layer "F.Cu") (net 7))
 (segment (start 137.16 98.044) (end 138.174 98.044) (width 0.3) (layer "F.Cu") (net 7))
 (segment (start 138.174 98.044) (end 138.176 98.042) (width 0.3) (layer "F.Cu") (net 7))
 (segment (start 135.636 97.4325) (end 136.5485 97.4325) (width 0.3) (layer "F.Cu") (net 7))
 (segment (start 142.24 99.568) (end 142.494 99.314) (width 0.3) (layer "F.Cu") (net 8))
 (segment (start 141.704 99.568) (end 142.24 99.568) (width 0.3) (layer "F.Cu") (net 8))
 (segment (start 142.494 99.314) (end 143.609 99.314) (width 0.3) (layer "F.Cu") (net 8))
 (segment (start 143.609 99.314) (end 143.64 99.345) (width 0.3) (layer "F.Cu") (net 8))
 (segment (start 148.64 94.265) (end 149.956 94.265) (width 0.25) (layer "F.Cu") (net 14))
 (segment (start 152.893 93.726) (end 154.671 95.504) (width 0.25) (layer "F.Cu") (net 14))
 (segment (start 150.495 93.726) (end 152.893 93.726) (width 0.25) (layer "F.Cu") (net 14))
 (segment (start 149.956 94.265) (end 150.495 93.726) (width 0.25) (layer "F.Cu") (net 14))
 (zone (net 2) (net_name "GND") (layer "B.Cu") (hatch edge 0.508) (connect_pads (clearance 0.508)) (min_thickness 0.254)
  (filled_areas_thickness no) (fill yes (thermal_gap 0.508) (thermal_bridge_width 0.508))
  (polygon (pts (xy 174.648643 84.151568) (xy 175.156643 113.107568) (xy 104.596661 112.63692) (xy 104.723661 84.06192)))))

